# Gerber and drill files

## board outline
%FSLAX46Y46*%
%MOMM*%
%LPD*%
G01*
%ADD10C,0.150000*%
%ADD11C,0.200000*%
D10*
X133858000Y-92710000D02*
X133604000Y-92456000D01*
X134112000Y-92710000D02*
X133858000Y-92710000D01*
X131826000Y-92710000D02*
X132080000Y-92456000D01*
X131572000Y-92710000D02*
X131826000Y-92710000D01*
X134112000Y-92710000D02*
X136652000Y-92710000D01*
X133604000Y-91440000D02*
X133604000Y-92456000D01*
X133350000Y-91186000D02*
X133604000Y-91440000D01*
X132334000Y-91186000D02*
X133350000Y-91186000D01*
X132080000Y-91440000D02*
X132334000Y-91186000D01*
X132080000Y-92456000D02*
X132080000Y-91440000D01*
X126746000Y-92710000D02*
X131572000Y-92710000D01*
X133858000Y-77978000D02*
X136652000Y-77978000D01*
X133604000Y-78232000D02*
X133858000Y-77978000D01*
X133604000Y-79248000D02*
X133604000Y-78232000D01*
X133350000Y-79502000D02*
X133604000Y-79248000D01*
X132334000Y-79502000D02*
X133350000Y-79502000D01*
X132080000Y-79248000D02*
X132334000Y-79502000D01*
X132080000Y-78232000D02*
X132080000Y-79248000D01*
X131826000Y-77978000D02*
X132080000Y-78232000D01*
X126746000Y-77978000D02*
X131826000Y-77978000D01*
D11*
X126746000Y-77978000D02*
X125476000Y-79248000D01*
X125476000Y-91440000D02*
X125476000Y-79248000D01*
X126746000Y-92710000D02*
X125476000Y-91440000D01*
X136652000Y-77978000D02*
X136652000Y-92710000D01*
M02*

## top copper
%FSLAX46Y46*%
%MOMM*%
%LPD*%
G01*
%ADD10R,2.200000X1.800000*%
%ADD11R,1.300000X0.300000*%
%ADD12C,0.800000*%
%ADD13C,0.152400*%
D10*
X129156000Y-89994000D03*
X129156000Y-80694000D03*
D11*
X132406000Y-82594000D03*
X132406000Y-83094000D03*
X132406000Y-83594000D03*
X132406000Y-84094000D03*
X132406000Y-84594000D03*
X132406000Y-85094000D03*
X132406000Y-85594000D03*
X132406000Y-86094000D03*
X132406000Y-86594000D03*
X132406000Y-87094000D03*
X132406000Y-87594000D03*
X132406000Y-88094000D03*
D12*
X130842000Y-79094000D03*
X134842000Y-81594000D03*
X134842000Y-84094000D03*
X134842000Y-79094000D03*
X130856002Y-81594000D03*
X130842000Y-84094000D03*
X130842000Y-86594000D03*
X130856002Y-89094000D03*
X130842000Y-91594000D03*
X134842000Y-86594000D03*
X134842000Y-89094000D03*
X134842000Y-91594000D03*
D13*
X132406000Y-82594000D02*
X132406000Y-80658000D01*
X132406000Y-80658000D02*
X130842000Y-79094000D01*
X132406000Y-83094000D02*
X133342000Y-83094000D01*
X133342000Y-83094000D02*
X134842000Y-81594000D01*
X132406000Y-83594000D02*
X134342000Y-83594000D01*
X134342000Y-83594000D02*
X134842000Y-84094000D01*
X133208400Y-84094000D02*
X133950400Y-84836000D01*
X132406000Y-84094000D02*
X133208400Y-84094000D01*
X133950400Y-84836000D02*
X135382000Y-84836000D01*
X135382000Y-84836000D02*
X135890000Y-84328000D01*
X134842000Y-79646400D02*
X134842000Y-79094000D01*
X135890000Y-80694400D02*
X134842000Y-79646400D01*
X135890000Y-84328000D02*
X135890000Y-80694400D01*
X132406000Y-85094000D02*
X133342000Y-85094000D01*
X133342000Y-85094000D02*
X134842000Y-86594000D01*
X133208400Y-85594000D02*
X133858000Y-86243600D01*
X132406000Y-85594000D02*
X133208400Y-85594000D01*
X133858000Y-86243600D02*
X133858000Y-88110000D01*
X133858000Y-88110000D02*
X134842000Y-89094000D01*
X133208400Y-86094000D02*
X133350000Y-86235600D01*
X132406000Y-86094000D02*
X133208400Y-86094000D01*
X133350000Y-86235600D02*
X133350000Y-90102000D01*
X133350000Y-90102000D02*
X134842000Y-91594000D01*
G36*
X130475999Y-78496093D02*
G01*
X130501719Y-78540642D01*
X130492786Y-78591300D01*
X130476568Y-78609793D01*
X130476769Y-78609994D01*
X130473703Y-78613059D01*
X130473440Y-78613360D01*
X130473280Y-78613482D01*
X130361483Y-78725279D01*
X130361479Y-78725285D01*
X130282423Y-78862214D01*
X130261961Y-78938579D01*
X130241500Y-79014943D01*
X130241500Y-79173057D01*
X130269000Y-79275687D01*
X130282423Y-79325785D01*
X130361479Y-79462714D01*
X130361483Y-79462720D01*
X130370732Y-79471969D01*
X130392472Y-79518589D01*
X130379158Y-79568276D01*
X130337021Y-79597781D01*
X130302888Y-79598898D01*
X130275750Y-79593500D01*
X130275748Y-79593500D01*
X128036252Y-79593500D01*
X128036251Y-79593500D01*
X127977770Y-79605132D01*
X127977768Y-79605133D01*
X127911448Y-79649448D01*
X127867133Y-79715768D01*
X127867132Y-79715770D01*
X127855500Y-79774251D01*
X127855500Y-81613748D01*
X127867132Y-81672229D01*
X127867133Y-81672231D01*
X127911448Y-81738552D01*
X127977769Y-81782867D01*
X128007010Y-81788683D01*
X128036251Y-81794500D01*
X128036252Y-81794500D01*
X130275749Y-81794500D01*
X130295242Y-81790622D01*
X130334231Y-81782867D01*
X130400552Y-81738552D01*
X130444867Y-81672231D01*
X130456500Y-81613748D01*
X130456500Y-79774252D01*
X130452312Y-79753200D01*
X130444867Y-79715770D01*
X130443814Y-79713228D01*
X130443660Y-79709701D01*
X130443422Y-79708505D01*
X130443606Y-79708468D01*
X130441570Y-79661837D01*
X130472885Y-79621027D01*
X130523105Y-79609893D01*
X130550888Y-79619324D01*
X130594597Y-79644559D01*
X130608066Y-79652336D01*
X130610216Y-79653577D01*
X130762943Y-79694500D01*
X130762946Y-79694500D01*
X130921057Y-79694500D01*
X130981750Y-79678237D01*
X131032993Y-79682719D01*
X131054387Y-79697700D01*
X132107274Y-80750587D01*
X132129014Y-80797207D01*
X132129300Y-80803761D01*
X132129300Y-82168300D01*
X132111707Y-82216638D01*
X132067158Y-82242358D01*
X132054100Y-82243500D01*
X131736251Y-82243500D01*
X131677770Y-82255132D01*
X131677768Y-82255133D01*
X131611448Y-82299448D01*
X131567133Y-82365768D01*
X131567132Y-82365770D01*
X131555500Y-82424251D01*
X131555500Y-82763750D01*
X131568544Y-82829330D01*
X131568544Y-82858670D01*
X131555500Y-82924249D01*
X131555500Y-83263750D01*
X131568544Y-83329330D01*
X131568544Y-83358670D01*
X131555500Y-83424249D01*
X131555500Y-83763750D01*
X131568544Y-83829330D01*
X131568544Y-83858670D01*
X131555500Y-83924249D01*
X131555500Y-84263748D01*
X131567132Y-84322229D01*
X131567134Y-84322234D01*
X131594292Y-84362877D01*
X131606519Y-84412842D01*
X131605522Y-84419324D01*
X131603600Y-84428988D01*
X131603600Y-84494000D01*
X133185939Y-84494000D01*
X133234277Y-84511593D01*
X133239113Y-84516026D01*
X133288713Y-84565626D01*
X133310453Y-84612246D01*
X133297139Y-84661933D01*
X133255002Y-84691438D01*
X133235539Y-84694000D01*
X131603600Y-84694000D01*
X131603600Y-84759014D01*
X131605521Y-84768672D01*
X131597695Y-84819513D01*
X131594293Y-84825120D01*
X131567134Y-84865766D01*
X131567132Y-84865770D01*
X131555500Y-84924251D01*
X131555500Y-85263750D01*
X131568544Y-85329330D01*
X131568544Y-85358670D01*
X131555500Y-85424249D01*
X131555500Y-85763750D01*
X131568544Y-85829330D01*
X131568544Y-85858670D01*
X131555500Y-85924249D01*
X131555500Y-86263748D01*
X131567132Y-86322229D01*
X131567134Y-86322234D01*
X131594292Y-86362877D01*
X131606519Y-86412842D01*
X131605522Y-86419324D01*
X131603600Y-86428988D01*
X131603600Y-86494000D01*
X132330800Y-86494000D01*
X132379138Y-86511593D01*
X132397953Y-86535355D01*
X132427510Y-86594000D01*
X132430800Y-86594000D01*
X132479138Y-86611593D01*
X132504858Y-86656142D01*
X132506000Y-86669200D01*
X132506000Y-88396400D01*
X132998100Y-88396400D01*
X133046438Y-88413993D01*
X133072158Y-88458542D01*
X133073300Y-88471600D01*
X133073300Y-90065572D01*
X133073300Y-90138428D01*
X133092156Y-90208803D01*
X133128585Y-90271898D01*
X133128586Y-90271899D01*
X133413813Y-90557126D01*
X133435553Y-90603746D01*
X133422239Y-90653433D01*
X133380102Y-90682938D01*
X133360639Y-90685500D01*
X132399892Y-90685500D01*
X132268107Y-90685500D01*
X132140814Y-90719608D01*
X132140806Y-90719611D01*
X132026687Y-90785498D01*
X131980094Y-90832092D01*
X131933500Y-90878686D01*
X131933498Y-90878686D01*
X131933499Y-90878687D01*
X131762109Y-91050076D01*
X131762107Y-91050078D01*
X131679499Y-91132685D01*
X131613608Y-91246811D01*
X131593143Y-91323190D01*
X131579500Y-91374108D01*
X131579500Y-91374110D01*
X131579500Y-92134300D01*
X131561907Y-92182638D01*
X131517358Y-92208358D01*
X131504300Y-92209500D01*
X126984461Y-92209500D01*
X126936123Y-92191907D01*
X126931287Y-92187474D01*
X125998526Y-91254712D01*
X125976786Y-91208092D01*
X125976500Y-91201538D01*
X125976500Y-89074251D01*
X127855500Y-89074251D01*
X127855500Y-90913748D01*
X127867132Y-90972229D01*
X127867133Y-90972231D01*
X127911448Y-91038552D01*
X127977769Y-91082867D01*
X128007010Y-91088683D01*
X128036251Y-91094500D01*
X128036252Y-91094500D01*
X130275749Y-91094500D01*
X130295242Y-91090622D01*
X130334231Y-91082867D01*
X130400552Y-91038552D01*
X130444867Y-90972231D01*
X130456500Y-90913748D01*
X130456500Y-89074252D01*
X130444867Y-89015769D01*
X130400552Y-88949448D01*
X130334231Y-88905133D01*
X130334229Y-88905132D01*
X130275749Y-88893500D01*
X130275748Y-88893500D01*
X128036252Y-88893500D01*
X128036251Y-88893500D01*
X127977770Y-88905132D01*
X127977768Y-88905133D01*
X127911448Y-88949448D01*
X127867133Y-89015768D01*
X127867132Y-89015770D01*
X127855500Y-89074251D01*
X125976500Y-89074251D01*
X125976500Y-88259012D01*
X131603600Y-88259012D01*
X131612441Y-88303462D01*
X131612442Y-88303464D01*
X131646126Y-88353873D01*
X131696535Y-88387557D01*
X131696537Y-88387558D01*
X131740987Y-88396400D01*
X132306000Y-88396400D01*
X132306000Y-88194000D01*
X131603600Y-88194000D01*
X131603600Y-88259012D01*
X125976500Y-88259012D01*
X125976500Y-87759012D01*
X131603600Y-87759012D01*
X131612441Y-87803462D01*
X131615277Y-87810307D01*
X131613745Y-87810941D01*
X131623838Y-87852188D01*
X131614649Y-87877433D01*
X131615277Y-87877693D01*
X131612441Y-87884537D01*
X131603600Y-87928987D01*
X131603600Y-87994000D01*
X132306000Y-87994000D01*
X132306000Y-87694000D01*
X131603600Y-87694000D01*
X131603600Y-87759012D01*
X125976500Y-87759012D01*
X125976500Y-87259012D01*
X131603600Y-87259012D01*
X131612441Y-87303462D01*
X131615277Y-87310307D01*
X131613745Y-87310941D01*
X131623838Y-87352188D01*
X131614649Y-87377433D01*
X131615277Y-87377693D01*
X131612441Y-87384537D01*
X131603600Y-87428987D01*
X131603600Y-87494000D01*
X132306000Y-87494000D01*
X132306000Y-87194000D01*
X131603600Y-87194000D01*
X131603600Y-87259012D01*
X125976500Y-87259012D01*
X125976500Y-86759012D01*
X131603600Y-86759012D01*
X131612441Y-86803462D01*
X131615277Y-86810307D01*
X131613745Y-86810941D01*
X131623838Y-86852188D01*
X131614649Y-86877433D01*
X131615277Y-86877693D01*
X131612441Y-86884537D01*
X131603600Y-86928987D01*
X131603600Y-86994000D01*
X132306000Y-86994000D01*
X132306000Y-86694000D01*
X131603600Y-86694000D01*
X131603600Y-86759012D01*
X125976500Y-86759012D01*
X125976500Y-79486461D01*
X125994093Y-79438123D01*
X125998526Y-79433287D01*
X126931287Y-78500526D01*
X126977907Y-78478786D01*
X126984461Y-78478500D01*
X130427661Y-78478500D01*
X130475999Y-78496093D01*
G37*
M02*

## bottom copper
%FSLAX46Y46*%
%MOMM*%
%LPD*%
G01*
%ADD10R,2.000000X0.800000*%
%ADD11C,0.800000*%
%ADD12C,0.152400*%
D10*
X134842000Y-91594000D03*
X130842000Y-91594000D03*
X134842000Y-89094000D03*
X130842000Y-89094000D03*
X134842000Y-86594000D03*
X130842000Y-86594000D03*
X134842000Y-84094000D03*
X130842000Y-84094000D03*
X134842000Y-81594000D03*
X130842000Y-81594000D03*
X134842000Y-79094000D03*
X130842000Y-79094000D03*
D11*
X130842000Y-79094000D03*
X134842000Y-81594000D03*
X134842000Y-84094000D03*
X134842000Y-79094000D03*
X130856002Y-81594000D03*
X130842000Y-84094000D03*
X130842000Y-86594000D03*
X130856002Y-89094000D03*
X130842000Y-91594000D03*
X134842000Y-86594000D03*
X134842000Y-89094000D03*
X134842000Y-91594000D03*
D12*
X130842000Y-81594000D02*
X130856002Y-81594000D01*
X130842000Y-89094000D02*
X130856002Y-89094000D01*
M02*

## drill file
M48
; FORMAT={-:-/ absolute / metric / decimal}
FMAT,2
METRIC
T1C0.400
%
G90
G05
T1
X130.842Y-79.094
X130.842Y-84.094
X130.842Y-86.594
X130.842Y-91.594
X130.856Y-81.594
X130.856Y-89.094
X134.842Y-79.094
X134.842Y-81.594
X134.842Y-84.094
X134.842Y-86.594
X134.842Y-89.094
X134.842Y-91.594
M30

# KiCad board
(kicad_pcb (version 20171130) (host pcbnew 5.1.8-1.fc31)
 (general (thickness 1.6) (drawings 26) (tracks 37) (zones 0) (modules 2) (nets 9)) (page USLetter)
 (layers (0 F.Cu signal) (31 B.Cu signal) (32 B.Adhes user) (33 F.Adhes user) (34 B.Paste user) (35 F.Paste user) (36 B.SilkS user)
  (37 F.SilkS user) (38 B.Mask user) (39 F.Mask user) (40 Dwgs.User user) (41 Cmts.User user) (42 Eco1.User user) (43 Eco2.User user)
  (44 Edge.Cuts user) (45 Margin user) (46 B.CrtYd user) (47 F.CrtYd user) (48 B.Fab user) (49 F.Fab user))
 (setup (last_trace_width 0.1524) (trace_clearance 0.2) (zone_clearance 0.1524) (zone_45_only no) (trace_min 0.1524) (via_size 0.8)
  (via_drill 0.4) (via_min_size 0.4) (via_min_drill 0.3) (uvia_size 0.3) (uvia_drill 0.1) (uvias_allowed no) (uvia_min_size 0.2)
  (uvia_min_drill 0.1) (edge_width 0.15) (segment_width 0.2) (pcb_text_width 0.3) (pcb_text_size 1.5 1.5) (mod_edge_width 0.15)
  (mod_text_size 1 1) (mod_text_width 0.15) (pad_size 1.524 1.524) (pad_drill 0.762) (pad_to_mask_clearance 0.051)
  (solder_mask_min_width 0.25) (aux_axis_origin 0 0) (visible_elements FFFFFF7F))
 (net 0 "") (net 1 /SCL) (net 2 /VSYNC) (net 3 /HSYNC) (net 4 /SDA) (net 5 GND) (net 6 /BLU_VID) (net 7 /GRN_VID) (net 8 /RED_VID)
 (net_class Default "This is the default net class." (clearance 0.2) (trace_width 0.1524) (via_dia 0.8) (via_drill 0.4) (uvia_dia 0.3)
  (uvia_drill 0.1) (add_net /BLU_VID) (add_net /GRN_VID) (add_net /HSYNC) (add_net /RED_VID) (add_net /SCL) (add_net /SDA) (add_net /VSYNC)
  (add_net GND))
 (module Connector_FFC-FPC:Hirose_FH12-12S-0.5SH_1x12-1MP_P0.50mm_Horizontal (layer F.Cu) (at 130.556 85.344 270)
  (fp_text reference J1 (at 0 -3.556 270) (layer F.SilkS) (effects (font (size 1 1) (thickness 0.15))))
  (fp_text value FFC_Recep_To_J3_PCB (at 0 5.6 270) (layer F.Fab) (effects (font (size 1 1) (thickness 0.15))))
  (pad MP smd rect (at 4.65 1.4 270) (size 1.8 2.2) (layers F.Cu F.Paste F.Mask))
  (pad MP smd rect (at -4.65 1.4 270) (size 1.8 2.2) (layers F.Cu F.Paste F.Mask))
  (pad 1 smd rect (at -2.75 -1.85 270) (size 0.3 1.3) (layers F.Cu F.Paste F.Mask) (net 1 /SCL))
  (pad 2 smd rect (at -2.25 -1.85 270) (size 0.3 1.3) (layers F.Cu F.Paste F.Mask) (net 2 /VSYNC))
  (pad 3 smd rect (at -1.75 -1.85 270) (size 0.3 1.3) (layers F.Cu F.Paste F.Mask) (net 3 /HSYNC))
  (pad 4 smd rect (at -1.25 -1.85 270) (size 0.3 1.3) (layers F.Cu F.Paste F.Mask) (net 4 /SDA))
  (pad 5 smd rect (at -0.75 -1.85 270) (size 0.3 1.3) (layers F.Cu F.Paste F.Mask) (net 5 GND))
  (pad 6 smd rect (at -0.25 -1.85 270) (size 0.3 1.3) (layers F.Cu F.Paste F.Mask) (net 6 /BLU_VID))
  (pad 7 smd rect (at 0.25 -1.85 270) (size 0.3 1.3) (layers F.Cu F.Paste F.Mask) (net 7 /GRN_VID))
  (pad 8 smd rect (at 0.75 -1.85 270) (size 0.3 1.3) (layers F.Cu F.Paste F.Mask) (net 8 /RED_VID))
  (pad 9 smd rect (at 1.25 -1.85 270) (size 0.3 1.3) (layers F.Cu F.Paste F.Mask) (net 5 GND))
  (pad 10 smd rect (at 1.75 -1.85 270) (size 0.3 1.3) (layers F.Cu F.Paste F.Mask) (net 5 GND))
  (pad 11 smd rect (at 2.25 -1.85 270) (size 0.3 1.3) (layers F.Cu F.Paste F.Mask) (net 5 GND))
  (pad 12 smd rect (at 2.75 -1.85 270) (size 0.3 1.3) (layers F.Cu F.Paste F.Mask) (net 5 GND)))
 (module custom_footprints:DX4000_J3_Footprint (layer B.Cu) (at 132.842 85.344)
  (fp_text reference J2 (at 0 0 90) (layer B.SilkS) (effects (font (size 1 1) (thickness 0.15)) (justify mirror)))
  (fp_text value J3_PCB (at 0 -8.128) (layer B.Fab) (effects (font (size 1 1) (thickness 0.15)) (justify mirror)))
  (pad 1 smd rect (at 2 6.25) (size 2 0.8) (layers B.Cu B.Paste B.Mask) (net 8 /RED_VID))
  (pad 2 smd rect (at -2 6.25) (size 2 0.8) (layers B.Cu B.Paste B.Mask) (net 5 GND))
  (pad 3 smd rect (at 2 3.75) (size 2 0.8) (layers B.Cu B.Paste B.Mask) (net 7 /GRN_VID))
  (pad 4 smd rect (at -2 3.75) (size 2 0.8) (layers B.Cu B.Paste B.Mask) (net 5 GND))
  (pad 5 smd rect (at 2 1.25) (size 2 0.8) (layers B.Cu B.Paste B.Mask) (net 6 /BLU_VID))
  (pad 6 smd rect (at -2 1.25) (size 2 0.8) (layers B.Cu B.Paste B.Mask) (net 5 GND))
  (pad 7 smd rect (at 2 -1.25) (size 2 0.8) (layers B.Cu B.Paste B.Mask) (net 3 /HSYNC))
  (pad 8 smd rect (at -2 -1.25) (size 2 0.8) (layers B.Cu B.Paste B.Mask) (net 5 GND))
  (pad 9 smd rect (at 2 -3.75) (size 2 0.8) (layers B.Cu B.Paste B.Mask) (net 2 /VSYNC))
  (pad 10 smd rect (at -2 -3.75) (size 2 0.8) (layers B.Cu B.Paste B.Mask) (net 5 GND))
  (pad 11 smd rect (at 2 -6.25) (size 2 0.8) (layers B.Cu B.Paste B.Mask) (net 4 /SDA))
  (pad 12 smd rect (at -2 -6.25) (size 2 0.8) (layers B.Cu B.Paste B.Mask) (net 1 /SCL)))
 (gr_line (start 133.858 92.71) (end 133.604 92.456) (layer Edge.Cuts) (width 0.15))
 (gr_line (start 134.112 92.71) (end 133.858 92.71) (layer Edge.Cuts) (width 0.15))
 (gr_line (start 131.826 92.71) (end 132.08 92.456) (layer Edge.Cuts) (width 0.15))
 (gr_line (start 131.572 92.71) (end 131.826 92.71) (layer Edge.Cuts) (width 0.15))
 (gr_line (start 134.112 92.71) (end 136.652 92.71) (layer Edge.Cuts) (width 0.15))
 (gr_line (start 133.604 91.44) (end 133.604 92.456) (layer Edge.Cuts) (width 0.15))
 (gr_line (start 133.35 91.186) (end 133.604 91.44) (layer Edge.Cuts) (width 0.15))
 (gr_line (start 132.334 91.186) (end 133.35 91.186) (layer Edge.Cuts) (width 0.15))
 (gr_line (start 132.08 91.44) (end 132.334 91.186) (layer Edge.Cuts) (width 0.15))
 (gr_line (start 132.08 92.456) (end 132.08 91.44) (layer Edge.Cuts) (width 0.15))
 (gr_line (start 126.746 92.71) (end 131.572 92.71) (layer Edge.Cuts) (width 0.15))
 (gr_line (start 133.858 77.978) (end 136.652 77.978) (layer Edge.Cuts) (width 0.15))
 (gr_line (start 133.604 78.232) (end 133.858 77.978) (layer Edge.Cuts) (width 0.15))
 (gr_line (start 133.604 79.248) (end 133.604 78.232) (layer Edge.Cuts) (width 0.15))
 (gr_line (start 133.35 79.502) (end 133.604 79.248) (layer Edge.Cuts) (width 0.15))
 (gr_line (start 132.334 79.502) (end 133.35 79.502) (layer Edge.Cuts) (width 0.15))
 (gr_line (start 132.08 79.248) (end 132.334 79.502) (layer Edge.Cuts) (width 0.15))
 (gr_line (start 132.08 78.232) (end 132.08 79.248) (layer Edge.Cuts) (width 0.15))
 (gr_line (start 131.826 77.978) (end 132.08 78.232) (layer Edge.Cuts) (width 0.15))
 (gr_line (start 126.746 77.978) (end 131.826 77.978) (layer Edge.Cuts) (width 0.15))
 (gr_line (start 126.746 77.978) (end 125.476 79.248) (layer Edge.Cuts) (width 0.2))
 (gr_line (start 125.476 91.44) (end 125.476 79.248) (layer Edge.Cuts) (width 0.2))
 (gr_line (start 126.746 92.71) (end 125.476 91.44) (layer Edge.Cuts) (width 0.2))
 (gr_line (start 136.652 77.978) (end 136.652 92.71) (layer Edge.Cuts) (width 0.2))
 (via (at 130.842 79.094) (size 0.8) (drill 0.4) (layers F.Cu B.Cu) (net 1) (status 30))
 (segment (start 132.406 82.594) (end 132.406 80.658) (width 0.1524) (layer F.Cu) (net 1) (status 10))
 (segment (start 132.406 80.658) (end 130.842 79.094) (width 0.1524) (layer F.Cu) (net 1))
 (via (at 134.842 81.594) (size 0.8) (drill 0.4) (layers F.Cu B.Cu) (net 2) (status 30))
 (segment (start 132.406 83.094) (end 133.342 83.094) (width 0.1524) (layer F.Cu) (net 2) (status 10))
 (segment (start 133.342 83.094) (end 134.842 81.594) (width 0.1524) (layer F.Cu) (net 2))
 (via (at 134.842 84.094) (size 0.8) (drill 0.4) (layers F.Cu B.Cu) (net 3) (status 30))
 (segment (start 132.406 83.594) (end 134.342 83.594) (width 0.1524) (layer F.Cu) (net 3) (status 10))
 (segment (start 134.342 83.594) (end 134.842 84.094) (width 0.1524) (layer F.Cu) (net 3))
 (via (at 134.842 79.094) (size 0.8) (drill 0.4) (layers F.Cu B.Cu) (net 4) (status 30))
 (segment (start 133.2084 84.094) (end 133.9504 84.836) (width 0.1524) (layer F.Cu) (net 4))
 (segment (start 132.406 84.094) (end 133.2084 84.094) (width 0.1524) (layer F.Cu) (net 4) (status 10))
 (segment (start 133.9504 84.836) (end 135.382 84.836) (width 0.1524) (layer F.Cu) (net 4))
 (segment (start 135.382 84.836) (end 135.89 84.328) (width 0.1524) (layer F.Cu) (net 4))
 (segment (start 134.842 79.6464) (end 134.842 79.094) (width 0.1524) (layer F.Cu) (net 4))
 (segment (start 135.89 80.6944) (end 134.842 79.6464) (width 0.1524) (layer F.Cu) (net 4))
 (segment (start 135.89 84.328) (end 135.89 80.6944) (width 0.1524) (layer F.Cu) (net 4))
 (via (at 130.856002 81.594) (size 0.8) (drill 0.4) (layers F.Cu B.Cu) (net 5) (status 30))
 (segment (start 130.842 81.594) (end 130.856002 81.594) (width 0.1524) (layer B.Cu) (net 5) (status 30))
 (via (at 130.842 84.094) (size 0.8) (drill 0.4) (layers F.Cu B.Cu) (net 5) (status 30))
 (via (at 130.842 86.594) (size 0.8) (drill 0.4) (layers F.Cu B.Cu) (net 5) (status 30))
 (via (at 130.856002 89.094) (size 0.8) (drill 0.4) (layers F.Cu B.Cu) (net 5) (status 30))
 (segment (start 130.842 89.094) (end 130.856002 89.094) (width 0.1524) (layer B.Cu) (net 5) (status 30))
 (via (at 130.842 91.594) (size 0.8) (drill 0.4) (layers F.Cu B.Cu) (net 5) (status 30))
 (via (at 134.842 86.594) (size 0.8) (drill 0.4) (layers F.Cu B.Cu) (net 6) (status 30))
 (segment (start 132.406 85.094) (end 133.342 85.094) (width 0.1524) (layer F.Cu) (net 6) (status 10))
 (segment (start 133.342 85.094) (end 134.842 86.594) (width 0.1524) (layer F.Cu) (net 6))
 (segment (start 133.2084 85.594) (end 133.858 86.2436) (width 0.1524) (layer F.Cu) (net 7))
 (segment (start 132.406 85.594) (end 133.2084 85.594) (width 0.1524) (layer F.Cu) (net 7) (status 10))
 (via (at 134.842 89.094) (size 0.8) (drill 0.4) (layers F.Cu B.Cu) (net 7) (status 30))
 (segment (start 133.858 86.2436) (end 133.858 88.11) (width 0.1524) (layer F.Cu) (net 7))
 (segment (start 133.858 88.11) (end 134.842 89.094) (width 0.1524) (layer F.Cu) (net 7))
 (segment (start 133.2084 86.094) (end 133.35 86.2356) (width 0.1524) (layer F.Cu) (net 8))
 (segment (start 132.406 86.094) (end 133.2084 86.094) (width 0.1524) (layer F.Cu) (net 8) (status 10))
 (via (at 134.842 91.594) (size 0.8) (drill 0.4) (layers F.Cu B.Cu) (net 8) (status 30))
 (segment (start 133.35 86.2356) (end 133.35 90.102) (width 0.1524) (layer F.Cu) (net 8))
 (segment (start 133.35 90.102) (end 134.842 91.594) (width 0.1524) (layer F.Cu) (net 8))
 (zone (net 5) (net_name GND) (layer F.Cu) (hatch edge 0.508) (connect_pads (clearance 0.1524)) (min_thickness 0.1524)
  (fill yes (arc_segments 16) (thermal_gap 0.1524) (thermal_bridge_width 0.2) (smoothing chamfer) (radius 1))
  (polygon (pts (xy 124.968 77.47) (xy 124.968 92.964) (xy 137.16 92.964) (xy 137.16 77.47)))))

